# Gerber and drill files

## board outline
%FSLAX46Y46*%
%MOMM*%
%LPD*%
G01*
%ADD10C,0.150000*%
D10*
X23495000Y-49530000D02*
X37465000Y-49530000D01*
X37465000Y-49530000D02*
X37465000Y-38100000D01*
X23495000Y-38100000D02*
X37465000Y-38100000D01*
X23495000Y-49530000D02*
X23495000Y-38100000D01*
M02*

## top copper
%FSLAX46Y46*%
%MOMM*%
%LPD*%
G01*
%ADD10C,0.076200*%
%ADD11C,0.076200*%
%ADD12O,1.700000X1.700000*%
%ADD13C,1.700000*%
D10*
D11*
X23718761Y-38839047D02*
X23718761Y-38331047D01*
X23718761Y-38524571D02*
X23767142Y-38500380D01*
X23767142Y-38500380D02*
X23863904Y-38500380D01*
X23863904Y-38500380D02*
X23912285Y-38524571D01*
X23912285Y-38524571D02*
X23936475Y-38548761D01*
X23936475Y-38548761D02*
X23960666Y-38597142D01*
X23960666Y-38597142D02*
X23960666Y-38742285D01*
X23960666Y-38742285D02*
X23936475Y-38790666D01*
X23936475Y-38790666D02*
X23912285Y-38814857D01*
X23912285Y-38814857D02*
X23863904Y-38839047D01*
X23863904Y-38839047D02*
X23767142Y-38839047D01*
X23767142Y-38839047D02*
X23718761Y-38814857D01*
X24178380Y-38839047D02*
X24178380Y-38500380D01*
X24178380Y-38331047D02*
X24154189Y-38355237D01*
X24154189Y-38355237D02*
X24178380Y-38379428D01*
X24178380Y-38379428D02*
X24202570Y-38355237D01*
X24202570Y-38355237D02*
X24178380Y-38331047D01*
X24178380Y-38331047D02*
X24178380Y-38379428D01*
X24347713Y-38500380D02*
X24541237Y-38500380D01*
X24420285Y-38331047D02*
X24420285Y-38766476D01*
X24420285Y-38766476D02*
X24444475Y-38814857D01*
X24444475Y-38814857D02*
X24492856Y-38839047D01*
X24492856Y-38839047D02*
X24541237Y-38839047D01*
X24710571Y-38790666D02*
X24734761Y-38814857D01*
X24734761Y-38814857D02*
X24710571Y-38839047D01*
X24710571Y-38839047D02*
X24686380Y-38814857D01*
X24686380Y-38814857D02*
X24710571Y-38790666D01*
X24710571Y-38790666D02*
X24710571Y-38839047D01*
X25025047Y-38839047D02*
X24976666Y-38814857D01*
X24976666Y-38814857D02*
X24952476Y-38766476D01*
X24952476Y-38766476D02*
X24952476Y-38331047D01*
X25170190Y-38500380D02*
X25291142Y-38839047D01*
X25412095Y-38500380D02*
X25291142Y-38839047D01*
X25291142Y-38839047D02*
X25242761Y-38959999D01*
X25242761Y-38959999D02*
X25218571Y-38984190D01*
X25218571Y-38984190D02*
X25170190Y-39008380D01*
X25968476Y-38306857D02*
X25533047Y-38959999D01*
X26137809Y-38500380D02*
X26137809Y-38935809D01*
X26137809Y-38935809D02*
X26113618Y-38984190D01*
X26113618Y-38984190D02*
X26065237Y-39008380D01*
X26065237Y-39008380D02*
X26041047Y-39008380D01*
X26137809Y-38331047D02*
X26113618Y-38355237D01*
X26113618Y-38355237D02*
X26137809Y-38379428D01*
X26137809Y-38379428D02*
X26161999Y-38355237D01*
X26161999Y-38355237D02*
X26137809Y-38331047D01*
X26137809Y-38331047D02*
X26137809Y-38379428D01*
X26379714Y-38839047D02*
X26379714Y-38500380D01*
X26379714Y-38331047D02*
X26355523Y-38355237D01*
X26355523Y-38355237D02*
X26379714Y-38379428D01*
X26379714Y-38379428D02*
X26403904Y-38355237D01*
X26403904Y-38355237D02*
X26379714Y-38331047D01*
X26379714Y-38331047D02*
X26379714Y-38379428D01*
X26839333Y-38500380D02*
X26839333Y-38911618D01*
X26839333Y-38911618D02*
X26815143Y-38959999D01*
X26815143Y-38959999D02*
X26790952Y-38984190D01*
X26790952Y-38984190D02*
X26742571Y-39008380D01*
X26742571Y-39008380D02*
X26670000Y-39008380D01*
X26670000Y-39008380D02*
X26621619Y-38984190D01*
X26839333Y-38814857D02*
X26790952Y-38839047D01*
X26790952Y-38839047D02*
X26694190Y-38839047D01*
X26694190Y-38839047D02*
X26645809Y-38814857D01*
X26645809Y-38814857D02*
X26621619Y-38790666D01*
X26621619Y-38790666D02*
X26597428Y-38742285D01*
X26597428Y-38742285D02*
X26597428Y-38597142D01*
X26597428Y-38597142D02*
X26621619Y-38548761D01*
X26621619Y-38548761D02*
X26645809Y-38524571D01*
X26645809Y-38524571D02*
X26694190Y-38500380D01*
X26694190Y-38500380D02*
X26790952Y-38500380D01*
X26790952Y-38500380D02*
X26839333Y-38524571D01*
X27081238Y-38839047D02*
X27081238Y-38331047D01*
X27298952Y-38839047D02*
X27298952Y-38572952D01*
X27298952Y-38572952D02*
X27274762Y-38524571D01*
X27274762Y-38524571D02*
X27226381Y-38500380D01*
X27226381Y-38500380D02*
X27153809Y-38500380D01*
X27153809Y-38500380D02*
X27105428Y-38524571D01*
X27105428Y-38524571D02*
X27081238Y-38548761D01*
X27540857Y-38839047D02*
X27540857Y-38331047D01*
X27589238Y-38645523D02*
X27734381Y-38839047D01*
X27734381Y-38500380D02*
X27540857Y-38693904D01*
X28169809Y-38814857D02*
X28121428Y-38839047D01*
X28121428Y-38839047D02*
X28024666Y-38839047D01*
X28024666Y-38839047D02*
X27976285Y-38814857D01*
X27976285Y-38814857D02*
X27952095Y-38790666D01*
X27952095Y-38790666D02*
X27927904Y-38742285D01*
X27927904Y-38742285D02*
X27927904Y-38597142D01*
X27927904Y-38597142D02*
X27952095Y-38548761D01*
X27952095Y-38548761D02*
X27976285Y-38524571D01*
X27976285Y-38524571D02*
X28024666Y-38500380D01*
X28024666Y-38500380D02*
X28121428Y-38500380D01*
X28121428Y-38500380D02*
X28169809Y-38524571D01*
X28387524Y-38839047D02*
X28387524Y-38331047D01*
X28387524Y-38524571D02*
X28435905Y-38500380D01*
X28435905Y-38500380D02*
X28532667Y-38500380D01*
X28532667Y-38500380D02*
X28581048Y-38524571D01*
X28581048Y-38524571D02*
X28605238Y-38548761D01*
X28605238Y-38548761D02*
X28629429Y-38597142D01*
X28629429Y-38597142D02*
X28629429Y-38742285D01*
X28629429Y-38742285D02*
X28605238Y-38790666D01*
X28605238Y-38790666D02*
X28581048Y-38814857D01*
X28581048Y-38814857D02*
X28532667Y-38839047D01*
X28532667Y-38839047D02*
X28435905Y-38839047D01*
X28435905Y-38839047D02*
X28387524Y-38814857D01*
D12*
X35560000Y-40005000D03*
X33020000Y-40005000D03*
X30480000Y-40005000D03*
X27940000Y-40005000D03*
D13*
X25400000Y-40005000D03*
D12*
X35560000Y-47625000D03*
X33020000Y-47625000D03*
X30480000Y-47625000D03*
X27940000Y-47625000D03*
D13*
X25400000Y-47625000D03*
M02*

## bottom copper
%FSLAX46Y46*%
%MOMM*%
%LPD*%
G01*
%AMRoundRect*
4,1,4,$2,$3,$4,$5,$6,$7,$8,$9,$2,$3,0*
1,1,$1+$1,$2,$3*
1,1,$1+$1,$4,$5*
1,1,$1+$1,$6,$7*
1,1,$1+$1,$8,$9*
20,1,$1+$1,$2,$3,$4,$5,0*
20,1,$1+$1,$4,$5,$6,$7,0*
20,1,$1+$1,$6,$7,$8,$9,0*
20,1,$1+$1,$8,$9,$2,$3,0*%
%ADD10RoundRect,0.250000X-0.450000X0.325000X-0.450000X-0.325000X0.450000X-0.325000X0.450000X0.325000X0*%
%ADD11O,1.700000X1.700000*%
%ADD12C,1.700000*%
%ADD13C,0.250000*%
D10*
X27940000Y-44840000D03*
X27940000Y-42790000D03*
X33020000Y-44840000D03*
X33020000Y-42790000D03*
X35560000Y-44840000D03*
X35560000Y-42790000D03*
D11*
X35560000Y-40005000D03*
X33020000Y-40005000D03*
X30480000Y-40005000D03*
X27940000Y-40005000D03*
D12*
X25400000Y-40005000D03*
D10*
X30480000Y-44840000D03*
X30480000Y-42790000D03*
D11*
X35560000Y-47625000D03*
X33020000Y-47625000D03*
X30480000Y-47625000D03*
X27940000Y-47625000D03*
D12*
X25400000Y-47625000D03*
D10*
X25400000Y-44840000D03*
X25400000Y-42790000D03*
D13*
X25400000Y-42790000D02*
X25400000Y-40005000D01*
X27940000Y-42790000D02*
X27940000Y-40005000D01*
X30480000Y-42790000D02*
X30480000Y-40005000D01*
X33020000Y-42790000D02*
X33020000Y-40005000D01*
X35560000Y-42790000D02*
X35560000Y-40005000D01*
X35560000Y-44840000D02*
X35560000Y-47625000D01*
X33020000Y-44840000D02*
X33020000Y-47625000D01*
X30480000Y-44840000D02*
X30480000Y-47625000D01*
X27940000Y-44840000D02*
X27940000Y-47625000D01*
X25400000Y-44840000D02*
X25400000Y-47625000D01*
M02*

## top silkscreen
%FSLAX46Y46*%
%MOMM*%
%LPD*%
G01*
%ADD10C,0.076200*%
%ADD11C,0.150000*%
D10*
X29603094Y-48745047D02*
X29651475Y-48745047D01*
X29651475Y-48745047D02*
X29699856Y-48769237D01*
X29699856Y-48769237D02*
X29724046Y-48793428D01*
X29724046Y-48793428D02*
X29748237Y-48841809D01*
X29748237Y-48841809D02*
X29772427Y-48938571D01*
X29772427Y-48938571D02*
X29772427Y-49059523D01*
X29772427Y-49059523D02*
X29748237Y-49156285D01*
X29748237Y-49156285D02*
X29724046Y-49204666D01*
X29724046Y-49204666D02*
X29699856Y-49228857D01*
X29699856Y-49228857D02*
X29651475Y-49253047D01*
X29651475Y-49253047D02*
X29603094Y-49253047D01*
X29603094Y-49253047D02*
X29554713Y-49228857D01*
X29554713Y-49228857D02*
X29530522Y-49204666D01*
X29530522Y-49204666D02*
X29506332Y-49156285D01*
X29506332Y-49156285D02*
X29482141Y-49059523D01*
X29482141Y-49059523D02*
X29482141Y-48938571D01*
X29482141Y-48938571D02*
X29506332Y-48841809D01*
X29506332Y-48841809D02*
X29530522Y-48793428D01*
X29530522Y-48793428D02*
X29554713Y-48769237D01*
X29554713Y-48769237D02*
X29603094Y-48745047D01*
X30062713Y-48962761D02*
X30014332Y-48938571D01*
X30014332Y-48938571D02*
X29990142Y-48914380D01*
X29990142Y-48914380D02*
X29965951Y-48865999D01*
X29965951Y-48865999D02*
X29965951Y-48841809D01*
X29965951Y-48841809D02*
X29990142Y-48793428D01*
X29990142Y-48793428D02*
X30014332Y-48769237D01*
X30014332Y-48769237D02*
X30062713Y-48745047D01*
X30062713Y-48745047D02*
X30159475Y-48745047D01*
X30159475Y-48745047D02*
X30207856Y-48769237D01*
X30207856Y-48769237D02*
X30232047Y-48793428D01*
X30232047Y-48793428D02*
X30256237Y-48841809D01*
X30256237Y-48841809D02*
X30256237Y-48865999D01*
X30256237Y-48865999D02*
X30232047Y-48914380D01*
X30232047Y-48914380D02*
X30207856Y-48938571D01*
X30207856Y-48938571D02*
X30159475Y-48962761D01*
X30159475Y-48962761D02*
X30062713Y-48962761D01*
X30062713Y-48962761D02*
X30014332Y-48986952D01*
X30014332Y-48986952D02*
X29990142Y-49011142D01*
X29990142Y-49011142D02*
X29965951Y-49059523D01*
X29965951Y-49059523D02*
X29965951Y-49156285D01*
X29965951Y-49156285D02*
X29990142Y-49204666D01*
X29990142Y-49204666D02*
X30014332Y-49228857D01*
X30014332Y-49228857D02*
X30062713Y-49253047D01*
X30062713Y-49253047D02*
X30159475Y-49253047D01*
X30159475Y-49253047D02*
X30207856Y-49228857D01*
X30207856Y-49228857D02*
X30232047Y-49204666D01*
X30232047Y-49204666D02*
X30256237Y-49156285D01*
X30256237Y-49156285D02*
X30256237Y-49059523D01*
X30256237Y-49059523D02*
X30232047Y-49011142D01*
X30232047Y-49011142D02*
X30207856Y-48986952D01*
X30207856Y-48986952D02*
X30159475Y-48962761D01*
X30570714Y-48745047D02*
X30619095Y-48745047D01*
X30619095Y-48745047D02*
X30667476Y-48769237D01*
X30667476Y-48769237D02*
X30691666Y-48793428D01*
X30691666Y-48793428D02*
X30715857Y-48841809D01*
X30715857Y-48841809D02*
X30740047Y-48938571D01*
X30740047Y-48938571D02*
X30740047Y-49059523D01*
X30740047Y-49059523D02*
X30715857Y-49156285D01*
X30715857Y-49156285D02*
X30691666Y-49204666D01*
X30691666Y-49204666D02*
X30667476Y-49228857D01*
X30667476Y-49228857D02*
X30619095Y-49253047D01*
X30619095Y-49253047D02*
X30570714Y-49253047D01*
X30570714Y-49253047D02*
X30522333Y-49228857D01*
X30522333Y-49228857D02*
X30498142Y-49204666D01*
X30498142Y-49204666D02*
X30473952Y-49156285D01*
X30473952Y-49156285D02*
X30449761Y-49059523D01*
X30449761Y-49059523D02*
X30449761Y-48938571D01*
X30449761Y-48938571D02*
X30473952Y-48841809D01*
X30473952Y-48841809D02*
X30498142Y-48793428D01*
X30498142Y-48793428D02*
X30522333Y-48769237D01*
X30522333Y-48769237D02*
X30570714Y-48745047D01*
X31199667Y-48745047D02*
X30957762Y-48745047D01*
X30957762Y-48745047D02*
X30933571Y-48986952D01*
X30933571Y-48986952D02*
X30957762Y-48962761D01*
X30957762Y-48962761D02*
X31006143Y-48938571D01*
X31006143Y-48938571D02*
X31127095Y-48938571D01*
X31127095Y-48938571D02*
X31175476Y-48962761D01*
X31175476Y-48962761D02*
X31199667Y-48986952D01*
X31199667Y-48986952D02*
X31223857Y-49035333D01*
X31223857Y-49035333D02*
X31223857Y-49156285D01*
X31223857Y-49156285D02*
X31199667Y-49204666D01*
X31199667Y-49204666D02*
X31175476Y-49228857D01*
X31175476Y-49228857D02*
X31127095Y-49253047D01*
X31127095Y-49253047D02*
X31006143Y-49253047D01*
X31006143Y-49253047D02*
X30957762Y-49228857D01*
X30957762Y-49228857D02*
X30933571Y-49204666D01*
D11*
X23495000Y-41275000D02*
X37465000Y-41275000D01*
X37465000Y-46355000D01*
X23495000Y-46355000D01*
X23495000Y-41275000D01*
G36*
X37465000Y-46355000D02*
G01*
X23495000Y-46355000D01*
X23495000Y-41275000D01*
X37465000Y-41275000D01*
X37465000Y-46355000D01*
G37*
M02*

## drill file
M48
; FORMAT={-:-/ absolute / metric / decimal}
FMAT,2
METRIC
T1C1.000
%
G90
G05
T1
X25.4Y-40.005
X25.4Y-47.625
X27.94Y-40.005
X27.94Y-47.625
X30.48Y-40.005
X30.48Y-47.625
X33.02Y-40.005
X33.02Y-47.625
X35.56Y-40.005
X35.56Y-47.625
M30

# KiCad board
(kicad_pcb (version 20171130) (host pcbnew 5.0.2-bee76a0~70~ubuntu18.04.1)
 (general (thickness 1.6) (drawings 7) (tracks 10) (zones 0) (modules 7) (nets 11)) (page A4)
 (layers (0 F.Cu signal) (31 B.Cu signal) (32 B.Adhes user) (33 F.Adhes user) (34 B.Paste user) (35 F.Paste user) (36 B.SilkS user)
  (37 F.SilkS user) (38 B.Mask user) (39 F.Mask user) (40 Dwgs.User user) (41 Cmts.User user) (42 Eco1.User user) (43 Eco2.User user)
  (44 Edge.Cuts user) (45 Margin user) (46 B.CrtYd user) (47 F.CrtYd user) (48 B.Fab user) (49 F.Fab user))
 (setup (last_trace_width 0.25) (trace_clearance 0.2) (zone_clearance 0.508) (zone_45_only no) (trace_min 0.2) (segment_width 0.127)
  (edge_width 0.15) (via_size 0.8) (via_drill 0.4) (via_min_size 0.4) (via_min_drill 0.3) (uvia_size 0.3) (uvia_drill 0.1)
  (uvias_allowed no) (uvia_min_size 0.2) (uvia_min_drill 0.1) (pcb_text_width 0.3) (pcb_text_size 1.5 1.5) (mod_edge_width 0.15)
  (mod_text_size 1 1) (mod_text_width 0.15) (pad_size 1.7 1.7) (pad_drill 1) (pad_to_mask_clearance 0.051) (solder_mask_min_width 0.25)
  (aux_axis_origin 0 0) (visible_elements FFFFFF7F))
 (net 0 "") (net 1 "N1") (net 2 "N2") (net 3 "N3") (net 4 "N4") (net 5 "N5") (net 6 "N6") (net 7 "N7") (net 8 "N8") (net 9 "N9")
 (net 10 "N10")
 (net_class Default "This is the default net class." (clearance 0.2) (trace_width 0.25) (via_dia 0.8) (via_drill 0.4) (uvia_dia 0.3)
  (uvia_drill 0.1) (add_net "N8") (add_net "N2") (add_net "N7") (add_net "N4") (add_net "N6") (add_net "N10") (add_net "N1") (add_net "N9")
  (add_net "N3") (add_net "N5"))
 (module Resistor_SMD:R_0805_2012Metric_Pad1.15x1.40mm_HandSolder (layer B.Cu) (at 27.94 43.815 270)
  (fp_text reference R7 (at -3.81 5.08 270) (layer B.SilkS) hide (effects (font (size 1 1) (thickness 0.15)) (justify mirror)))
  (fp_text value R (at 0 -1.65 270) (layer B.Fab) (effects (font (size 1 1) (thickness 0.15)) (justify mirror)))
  (pad 2 smd roundrect (at 1.025 0 270) (size 1.15 1.4) (layers B.Cu B.Paste B.Mask) (roundrect_rratio 0.217391) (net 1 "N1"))
  (pad 1 smd roundrect (at -1.025 0 270) (size 1.15 1.4) (layers B.Cu B.Paste B.Mask) (roundrect_rratio 0.217391) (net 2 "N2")))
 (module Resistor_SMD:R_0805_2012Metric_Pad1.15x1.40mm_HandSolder (layer B.Cu) (at 33.02 43.815 270)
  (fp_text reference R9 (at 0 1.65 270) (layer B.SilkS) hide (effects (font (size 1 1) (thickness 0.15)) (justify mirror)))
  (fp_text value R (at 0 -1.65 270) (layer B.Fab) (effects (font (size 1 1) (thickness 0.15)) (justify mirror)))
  (pad 2 smd roundrect (at 1.025 0 270) (size 1.15 1.4) (layers B.Cu B.Paste B.Mask) (roundrect_rratio 0.217391) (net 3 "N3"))
  (pad 1 smd roundrect (at -1.025 0 270) (size 1.15 1.4) (layers B.Cu B.Paste B.Mask) (roundrect_rratio 0.217391) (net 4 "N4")))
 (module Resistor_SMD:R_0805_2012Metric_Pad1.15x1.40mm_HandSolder (layer B.Cu) (at 35.56 43.815 270)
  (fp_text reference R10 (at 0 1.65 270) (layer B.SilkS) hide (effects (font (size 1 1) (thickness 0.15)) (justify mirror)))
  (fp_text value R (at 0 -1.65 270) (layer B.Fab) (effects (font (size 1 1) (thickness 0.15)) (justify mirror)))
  (pad 2 smd roundrect (at 1.025 0 270) (size 1.15 1.4) (layers B.Cu B.Paste B.Mask) (roundrect_rratio 0.217391) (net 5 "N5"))
  (pad 1 smd roundrect (at -1.025 0 270) (size 1.15 1.4) (layers B.Cu B.Paste B.Mask) (roundrect_rratio 0.217391) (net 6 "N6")))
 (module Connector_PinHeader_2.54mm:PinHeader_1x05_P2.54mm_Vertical (layer B.Cu) (at 25.4 40.005 270)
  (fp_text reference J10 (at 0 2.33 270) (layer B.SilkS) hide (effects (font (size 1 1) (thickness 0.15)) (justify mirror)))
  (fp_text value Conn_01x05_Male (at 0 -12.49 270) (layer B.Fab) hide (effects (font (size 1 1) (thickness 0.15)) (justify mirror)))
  (pad 5 thru_hole oval (at 0 -10.16 270) (size 1.7 1.7) (drill 1) (layers *.Cu *.Mask) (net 6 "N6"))
  (pad 4 thru_hole oval (at 0 -7.62 270) (size 1.7 1.7) (drill 1) (layers *.Cu *.Mask) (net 4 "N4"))
  (pad 3 thru_hole oval (at 0 -5.08 270) (size 1.7 1.7) (drill 1) (layers *.Cu *.Mask) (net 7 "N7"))
  (pad 2 thru_hole oval (at 0 -2.54 270) (size 1.7 1.7) (drill 1) (layers *.Cu *.Mask) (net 2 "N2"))
  (pad 1 thru_hole circle (at 0 0 270) (size 1.7 1.7) (drill 1) (layers *.Cu *.Mask) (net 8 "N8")))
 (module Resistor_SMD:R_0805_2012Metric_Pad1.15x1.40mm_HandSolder (layer B.Cu) (at 30.48 43.815 270)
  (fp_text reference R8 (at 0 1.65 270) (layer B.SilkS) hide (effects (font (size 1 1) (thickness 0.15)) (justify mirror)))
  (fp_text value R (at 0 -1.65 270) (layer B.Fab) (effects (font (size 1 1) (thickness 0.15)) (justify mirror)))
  (pad 2 smd roundrect (at 1.025 0 270) (size 1.15 1.4) (layers B.Cu B.Paste B.Mask) (roundrect_rratio 0.217391) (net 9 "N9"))
  (pad 1 smd roundrect (at -1.025 0 270) (size 1.15 1.4) (layers B.Cu B.Paste B.Mask) (roundrect_rratio 0.217391) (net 7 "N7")))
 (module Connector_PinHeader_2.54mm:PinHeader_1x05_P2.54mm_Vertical (layer B.Cu) (at 25.4 47.625 270)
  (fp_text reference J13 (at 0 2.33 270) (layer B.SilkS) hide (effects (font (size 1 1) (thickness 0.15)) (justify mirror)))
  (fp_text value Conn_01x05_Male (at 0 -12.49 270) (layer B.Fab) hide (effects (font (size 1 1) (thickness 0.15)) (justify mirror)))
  (pad 5 thru_hole oval (at 0 -10.16 270) (size 1.7 1.7) (drill 1) (layers *.Cu *.Mask) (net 5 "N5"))
  (pad 4 thru_hole oval (at 0 -7.62 270) (size 1.7 1.7) (drill 1) (layers *.Cu *.Mask) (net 3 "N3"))
  (pad 3 thru_hole oval (at 0 -5.08 270) (size 1.7 1.7) (drill 1) (layers *.Cu *.Mask) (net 9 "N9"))
  (pad 2 thru_hole oval (at 0 -2.54 270) (size 1.7 1.7) (drill 1) (layers *.Cu *.Mask) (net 1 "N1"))
  (pad 1 thru_hole circle (at 0 0 270) (size 1.7 1.7) (drill 1) (layers *.Cu *.Mask) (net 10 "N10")))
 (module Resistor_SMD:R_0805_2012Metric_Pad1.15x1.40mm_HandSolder (layer B.Cu) (at 25.4 43.815 270)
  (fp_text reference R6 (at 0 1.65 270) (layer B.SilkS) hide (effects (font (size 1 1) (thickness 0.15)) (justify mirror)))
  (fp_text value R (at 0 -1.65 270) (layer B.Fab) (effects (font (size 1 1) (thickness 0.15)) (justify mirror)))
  (pad 2 smd roundrect (at 1.025 0 270) (size 1.15 1.4) (layers B.Cu B.Paste B.Mask) (roundrect_rratio 0.217391) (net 10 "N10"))
  (pad 1 smd roundrect (at -1.025 0 270) (size 1.15 1.4) (layers B.Cu B.Paste B.Mask) (roundrect_rratio 0.217391) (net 8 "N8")))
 (gr_line (start 23.495 49.53) (end 37.465 49.53) (layer Edge.Cuts) (width 0.15))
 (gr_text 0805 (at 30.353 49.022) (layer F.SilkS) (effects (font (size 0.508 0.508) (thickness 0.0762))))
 (gr_poly (pts (xy 23.495 41.275) (xy 37.465 41.275) (xy 37.465 46.355) (xy 23.495 46.355)) (layer F.SilkS) (width 0.15))
 (gr_line (start 37.465 49.53) (end 37.465 38.1) (layer Edge.Cuts) (width 0.15))
 (gr_line (start 23.495 38.1) (end 37.465 38.1) (layer Edge.Cuts) (width 0.15))
 (gr_line (start 23.495 49.53) (end 23.495 38.1) (layer Edge.Cuts) (width 0.15))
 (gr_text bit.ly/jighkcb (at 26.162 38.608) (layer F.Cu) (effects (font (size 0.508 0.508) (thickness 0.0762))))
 (segment (start 25.4 42.79) (end 25.4 40.005) (width 0.25) (layer B.Cu) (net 8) (status 30))
 (segment (start 27.94 42.79) (end 27.94 40.005) (width 0.25) (layer B.Cu) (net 2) (status 30))
 (segment (start 30.48 42.79) (end 30.48 40.005) (width 0.25) (layer B.Cu) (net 7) (status 30))
 (segment (start 33.02 42.79) (end 33.02 40.005) (width 0.25) (layer B.Cu) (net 4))
 (segment (start 35.56 42.79) (end 35.56 40.005) (width 0.25) (layer B.Cu) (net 6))
 (segment (start 35.56 44.84) (end 35.56 47.625) (width 0.25) (layer B.Cu) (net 5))
 (segment (start 33.02 44.84) (end 33.02 47.625) (width 0.25) (layer B.Cu) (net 3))
 (segment (start 30.48 44.84) (end 30.48 47.625) (width 0.25) (layer B.Cu) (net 9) (status 30))
 (segment (start 27.94 44.84) (end 27.94 47.625) (width 0.25) (layer B.Cu) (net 1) (status 30))
 (segment (start 25.4 44.84) (end 25.4 47.625) (width 0.25) (layer B.Cu) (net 10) (status 30)))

